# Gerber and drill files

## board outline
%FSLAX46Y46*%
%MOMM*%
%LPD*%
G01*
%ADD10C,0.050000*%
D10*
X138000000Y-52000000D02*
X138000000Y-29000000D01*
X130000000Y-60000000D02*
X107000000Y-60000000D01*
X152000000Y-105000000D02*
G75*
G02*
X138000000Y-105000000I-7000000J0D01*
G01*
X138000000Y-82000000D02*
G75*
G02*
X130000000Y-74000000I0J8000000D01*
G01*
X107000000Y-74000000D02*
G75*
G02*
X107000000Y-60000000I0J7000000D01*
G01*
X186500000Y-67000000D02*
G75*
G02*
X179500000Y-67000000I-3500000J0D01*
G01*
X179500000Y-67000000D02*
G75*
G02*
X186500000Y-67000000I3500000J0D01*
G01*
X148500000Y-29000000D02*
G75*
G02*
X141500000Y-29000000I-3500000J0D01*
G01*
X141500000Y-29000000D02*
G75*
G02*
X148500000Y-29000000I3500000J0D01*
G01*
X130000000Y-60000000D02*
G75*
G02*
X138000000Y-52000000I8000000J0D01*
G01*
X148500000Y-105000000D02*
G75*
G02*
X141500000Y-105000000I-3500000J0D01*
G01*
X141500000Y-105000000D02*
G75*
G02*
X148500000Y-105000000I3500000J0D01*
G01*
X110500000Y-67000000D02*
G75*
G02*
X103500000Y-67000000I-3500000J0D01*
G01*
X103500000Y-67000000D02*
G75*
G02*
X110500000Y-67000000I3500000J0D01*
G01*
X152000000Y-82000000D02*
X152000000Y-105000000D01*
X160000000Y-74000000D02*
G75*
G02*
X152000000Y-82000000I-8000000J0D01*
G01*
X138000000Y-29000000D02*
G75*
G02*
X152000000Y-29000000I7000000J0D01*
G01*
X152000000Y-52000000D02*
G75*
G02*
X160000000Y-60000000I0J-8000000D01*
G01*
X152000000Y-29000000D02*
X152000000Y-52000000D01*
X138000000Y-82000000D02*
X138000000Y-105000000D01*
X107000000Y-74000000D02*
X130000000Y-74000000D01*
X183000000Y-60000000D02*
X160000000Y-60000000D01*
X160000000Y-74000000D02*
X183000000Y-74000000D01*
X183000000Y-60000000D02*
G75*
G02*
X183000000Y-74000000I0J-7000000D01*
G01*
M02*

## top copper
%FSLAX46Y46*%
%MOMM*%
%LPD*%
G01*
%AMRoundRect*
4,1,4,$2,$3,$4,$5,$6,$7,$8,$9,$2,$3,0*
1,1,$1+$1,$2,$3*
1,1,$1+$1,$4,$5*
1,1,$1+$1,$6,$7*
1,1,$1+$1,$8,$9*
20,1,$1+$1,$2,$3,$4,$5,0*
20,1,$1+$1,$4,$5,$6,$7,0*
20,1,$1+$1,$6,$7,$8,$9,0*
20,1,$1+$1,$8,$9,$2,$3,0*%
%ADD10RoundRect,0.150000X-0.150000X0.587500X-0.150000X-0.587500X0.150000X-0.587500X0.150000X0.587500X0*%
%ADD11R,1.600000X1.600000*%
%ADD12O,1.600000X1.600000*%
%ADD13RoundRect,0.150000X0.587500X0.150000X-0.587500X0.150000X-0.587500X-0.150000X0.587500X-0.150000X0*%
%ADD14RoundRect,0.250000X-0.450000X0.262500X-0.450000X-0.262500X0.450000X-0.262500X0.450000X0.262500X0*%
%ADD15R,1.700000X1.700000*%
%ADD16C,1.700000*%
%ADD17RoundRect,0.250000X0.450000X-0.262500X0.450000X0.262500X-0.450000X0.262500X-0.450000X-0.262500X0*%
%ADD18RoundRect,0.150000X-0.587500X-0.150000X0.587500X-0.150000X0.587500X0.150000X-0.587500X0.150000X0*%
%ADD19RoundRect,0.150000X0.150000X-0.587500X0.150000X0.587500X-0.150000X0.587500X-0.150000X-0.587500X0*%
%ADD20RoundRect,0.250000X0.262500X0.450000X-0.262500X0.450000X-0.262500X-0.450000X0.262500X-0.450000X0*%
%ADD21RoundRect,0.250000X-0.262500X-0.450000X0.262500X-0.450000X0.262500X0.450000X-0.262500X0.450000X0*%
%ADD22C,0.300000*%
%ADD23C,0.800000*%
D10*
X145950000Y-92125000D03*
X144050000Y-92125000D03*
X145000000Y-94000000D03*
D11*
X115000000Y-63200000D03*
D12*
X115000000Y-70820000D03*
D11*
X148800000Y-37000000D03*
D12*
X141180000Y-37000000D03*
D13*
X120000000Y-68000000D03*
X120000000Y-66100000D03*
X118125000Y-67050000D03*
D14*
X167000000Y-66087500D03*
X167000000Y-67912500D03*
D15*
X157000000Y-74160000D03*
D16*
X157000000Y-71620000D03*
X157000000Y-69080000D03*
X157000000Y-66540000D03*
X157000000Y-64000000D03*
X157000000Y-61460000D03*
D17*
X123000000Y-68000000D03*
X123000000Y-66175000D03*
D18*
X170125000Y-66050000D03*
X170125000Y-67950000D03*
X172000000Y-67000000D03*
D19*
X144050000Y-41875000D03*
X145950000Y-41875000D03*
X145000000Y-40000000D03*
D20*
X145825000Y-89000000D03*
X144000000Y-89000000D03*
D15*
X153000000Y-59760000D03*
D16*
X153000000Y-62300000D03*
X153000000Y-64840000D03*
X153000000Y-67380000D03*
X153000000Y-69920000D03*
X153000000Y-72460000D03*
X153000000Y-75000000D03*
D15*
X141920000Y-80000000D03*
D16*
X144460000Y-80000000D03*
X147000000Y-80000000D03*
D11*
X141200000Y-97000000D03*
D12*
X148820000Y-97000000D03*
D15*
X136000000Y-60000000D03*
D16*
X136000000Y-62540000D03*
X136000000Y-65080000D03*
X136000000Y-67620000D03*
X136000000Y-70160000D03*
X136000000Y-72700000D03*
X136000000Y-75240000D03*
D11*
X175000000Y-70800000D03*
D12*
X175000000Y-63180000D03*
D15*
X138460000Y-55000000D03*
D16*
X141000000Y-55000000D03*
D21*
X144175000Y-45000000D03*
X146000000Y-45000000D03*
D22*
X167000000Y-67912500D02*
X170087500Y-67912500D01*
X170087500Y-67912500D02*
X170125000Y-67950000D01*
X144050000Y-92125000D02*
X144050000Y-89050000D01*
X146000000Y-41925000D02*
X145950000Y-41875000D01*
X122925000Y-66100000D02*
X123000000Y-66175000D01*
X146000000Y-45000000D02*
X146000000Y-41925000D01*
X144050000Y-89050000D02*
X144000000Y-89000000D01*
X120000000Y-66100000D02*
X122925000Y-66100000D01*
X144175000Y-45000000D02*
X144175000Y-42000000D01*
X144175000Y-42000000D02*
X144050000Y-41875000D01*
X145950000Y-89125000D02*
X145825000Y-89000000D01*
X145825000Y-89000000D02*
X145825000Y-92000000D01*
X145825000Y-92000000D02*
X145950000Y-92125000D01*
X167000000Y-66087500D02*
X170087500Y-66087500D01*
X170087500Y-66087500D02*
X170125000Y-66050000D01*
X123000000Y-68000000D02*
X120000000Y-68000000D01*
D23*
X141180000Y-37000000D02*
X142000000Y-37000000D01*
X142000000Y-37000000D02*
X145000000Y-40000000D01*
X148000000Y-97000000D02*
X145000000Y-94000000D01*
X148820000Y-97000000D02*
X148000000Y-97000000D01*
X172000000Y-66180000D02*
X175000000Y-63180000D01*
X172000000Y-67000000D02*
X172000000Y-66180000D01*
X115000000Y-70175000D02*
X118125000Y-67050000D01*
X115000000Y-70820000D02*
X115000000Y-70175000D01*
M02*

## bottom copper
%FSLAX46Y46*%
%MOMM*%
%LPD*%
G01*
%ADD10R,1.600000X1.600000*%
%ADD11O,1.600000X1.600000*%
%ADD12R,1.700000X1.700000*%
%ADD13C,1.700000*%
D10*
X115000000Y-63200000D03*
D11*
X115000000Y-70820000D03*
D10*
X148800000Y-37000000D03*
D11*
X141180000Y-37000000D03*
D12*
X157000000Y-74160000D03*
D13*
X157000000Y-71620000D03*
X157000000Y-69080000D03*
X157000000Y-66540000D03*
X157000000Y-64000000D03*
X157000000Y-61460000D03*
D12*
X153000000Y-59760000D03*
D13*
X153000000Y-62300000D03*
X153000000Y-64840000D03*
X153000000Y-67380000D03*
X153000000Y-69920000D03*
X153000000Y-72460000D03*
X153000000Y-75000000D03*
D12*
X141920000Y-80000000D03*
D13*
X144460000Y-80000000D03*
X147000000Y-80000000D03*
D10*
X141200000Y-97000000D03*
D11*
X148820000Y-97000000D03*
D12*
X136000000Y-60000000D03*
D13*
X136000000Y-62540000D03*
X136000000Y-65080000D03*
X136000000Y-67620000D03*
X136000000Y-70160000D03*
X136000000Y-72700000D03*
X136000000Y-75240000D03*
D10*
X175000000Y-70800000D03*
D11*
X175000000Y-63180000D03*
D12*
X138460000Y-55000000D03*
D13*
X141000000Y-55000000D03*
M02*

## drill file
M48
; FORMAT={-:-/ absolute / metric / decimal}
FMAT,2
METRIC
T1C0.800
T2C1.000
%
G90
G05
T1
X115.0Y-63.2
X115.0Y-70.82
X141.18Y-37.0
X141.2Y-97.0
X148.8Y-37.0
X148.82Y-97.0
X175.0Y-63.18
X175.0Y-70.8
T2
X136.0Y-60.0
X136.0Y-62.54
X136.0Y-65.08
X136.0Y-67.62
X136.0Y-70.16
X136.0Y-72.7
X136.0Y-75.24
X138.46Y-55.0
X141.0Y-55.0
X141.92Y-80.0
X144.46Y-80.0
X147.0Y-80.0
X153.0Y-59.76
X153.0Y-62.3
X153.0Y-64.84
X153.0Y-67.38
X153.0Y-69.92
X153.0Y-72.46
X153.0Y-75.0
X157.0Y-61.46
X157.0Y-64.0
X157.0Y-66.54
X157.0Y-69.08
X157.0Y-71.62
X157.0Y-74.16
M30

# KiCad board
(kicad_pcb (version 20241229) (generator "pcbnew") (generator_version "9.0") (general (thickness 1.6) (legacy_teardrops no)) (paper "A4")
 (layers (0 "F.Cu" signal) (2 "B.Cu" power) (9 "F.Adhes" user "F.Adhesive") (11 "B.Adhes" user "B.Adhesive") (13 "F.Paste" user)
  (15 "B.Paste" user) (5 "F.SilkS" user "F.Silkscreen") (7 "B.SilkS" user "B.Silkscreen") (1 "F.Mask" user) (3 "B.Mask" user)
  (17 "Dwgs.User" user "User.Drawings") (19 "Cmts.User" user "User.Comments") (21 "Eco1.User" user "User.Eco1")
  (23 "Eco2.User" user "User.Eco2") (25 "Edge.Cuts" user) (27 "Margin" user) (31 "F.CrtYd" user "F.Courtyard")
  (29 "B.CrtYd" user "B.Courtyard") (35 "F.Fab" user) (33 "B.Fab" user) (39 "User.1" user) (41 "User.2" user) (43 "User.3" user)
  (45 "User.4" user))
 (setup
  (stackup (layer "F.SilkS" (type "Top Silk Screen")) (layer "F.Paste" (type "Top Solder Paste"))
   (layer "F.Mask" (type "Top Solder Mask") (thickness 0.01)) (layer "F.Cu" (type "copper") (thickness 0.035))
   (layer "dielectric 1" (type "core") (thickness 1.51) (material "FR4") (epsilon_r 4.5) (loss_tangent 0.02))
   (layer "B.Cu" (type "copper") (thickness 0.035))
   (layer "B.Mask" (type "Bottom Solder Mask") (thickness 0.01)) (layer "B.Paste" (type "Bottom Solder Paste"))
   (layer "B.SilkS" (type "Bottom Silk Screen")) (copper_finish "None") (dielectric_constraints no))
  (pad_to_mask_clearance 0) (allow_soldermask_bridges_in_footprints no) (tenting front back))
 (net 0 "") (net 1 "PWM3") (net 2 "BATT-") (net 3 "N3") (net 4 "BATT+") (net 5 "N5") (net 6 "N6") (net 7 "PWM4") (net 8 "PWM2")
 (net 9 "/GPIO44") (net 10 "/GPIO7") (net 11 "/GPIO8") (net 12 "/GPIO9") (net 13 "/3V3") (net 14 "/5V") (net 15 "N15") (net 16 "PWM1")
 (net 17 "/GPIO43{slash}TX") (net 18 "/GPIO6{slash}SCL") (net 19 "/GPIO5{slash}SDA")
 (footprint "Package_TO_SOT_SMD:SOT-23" (layer "F.Cu") (at 145 93.0625 -90)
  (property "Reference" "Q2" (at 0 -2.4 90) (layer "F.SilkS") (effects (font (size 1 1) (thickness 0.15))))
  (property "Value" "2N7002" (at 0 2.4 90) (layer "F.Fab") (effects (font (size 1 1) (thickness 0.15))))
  (pad "1" smd roundrect (at -0.9375 -0.95 270) (size 1.475 0.6) (layers "F.Cu" "F.Mask" "F.Paste") (roundrect_rratio 0.25) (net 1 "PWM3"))
  (pad "2" smd roundrect (at -0.9375 0.95 270) (size 1.475 0.6) (layers "F.Cu" "F.Mask" "F.Paste") (roundrect_rratio 0.25) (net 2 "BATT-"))
  (pad "3" smd roundrect (at 0.9375 0 270) (size 1.475 0.6) (layers "F.Cu" "F.Mask" "F.Paste") (roundrect_rratio 0.25) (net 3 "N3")))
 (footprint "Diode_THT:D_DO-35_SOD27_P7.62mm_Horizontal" (layer "F.Cu") (at 115 63.2 -90)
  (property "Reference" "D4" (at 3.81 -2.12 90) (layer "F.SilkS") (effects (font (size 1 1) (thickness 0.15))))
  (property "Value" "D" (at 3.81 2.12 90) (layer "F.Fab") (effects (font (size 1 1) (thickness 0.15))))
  (pad "1" thru_hole rect (at 0 0 270) (size 1.6 1.6) (drill 0.8) (layers "*.Cu" "*.Mask") (remove_unused_layers no) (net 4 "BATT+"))
  (pad "2" thru_hole oval (at 7.62 0 270) (size 1.6 1.6) (drill 0.8) (layers "*.Cu" "*.Mask") (remove_unused_layers no) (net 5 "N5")))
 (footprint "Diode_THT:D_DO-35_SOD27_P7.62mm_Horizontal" (layer "F.Cu") (at 148.8 37 180)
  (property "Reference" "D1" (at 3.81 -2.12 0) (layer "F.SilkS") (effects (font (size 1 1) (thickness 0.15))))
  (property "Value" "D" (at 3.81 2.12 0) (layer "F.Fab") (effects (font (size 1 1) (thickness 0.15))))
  (pad "1" thru_hole rect (at 0 0 180) (size 1.6 1.6) (drill 0.8) (layers "*.Cu" "*.Mask") (remove_unused_layers no) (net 4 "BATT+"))
  (pad "2" thru_hole oval (at 7.62 0 180) (size 1.6 1.6) (drill 0.8) (layers "*.Cu" "*.Mask") (remove_unused_layers no) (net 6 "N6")))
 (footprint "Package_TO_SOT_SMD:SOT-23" (layer "F.Cu") (at 119.0625 67.05 180)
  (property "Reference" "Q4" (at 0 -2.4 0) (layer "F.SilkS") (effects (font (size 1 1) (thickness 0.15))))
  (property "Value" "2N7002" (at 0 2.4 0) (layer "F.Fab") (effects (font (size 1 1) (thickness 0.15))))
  (pad "1" smd roundrect (at -0.9375 -0.95 180) (size 1.475 0.6) (layers "F.Cu" "F.Mask" "F.Paste") (roundrect_rratio 0.25) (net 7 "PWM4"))
  (pad "2" smd roundrect (at -0.9375 0.95 180) (size 1.475 0.6) (layers "F.Cu" "F.Mask" "F.Paste") (roundrect_rratio 0.25) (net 2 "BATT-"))
  (pad "3" smd roundrect (at 0.9375 0 180) (size 1.475 0.6) (layers "F.Cu" "F.Mask" "F.Paste") (roundrect_rratio 0.25) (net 5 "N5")))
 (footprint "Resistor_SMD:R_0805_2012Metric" (layer "F.Cu") (at 167 67 -90)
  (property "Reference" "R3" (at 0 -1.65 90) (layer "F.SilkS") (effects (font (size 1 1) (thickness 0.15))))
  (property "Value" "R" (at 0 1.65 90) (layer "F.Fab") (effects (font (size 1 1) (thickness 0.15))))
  (pad "1" smd roundrect (at -0.9125 0 270) (size 1.025 1.4) (layers "F.Cu" "F.Mask" "F.Paste") (roundrect_rratio 0.243902) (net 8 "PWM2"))
  (pad "2" smd roundrect (at 0.9125 0 270) (size 1.025 1.4) (layers "F.Cu" "F.Mask" "F.Paste") (roundrect_rratio 0.243902) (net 2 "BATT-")))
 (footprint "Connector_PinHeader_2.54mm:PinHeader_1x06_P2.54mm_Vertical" (layer "F.Cu") (at 157 74.16 180)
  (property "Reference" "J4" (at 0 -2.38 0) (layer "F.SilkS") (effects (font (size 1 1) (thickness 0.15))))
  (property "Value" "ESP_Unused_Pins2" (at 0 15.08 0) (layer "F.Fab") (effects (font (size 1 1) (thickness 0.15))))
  (pad "1" thru_hole rect (at 0 0 180) (size 1.7 1.7) (drill 1) (layers "*.Cu" "*.Mask") (remove_unused_layers no) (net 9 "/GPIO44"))
  (pad "2" thru_hole circle (at 0 2.54 180) (size 1.7 1.7) (drill 1) (layers "*.Cu" "*.Mask") (remove_unused_layers no) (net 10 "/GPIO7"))
  (pad "3" thru_hole circle (at 0 5.08 180) (size 1.7 1.7) (drill 1) (layers "*.Cu" "*.Mask") (remove_unused_layers no) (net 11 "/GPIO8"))
  (pad "4" thru_hole circle (at 0 7.62 180) (size 1.7 1.7) (drill 1) (layers "*.Cu" "*.Mask") (remove_unused_layers no) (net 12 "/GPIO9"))
  (pad "5" thru_hole circle (at 0 10.16 180) (size 1.7 1.7) (drill 1) (layers "*.Cu" "*.Mask") (remove_unused_layers no) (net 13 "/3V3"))
  (pad "6" thru_hole circle (at 0 12.7 180) (size 1.7 1.7) (drill 1) (layers "*.Cu" "*.Mask") (remove_unused_layers no) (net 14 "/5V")))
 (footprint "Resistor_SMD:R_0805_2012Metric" (layer "F.Cu") (at 123 67.0875 90)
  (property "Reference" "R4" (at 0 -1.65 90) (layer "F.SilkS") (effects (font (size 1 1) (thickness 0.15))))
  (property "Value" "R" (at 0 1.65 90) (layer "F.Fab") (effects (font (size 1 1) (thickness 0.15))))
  (pad "1" smd roundrect (at -0.9125 0 90) (size 1.025 1.4) (layers "F.Cu" "F.Mask" "F.Paste") (roundrect_rratio 0.243902) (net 7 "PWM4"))
  (pad "2" smd roundrect (at 0.9125 0 90) (size 1.025 1.4) (layers "F.Cu" "F.Mask" "F.Paste") (roundrect_rratio 0.243902) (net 2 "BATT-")))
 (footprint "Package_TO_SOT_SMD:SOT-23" (layer "F.Cu") (at 171.0625 67)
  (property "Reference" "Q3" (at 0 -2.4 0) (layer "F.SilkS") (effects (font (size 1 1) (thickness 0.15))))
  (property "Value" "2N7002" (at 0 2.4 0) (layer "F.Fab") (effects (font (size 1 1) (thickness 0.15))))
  (pad "1" smd roundrect (at -0.9375 -0.95) (size 1.475 0.6) (layers "F.Cu" "F.Mask" "F.Paste") (roundrect_rratio 0.25) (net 8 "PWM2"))
  (pad "2" smd roundrect (at -0.9375 0.95) (size 1.475 0.6) (layers "F.Cu" "F.Mask" "F.Paste") (roundrect_rratio 0.25) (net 2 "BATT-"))
  (pad "3" smd roundrect (at 0.9375 0) (size 1.475 0.6) (layers "F.Cu" "F.Mask" "F.Paste") (roundrect_rratio 0.25) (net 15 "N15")))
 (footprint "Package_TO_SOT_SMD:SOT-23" (layer "F.Cu") (at 145 40.9375 90)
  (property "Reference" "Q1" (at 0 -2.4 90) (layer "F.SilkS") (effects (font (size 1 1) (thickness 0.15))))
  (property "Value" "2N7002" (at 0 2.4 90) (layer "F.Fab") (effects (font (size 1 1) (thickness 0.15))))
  (pad "1" smd roundrect (at -0.9375 -0.95 90) (size 1.475 0.6) (layers "F.Cu" "F.Mask" "F.Paste") (roundrect_rratio 0.25) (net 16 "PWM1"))
  (pad "2" smd roundrect (at -0.9375 0.95 90) (size 1.475 0.6) (layers "F.Cu" "F.Mask" "F.Paste") (roundrect_rratio 0.25) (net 2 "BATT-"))
  (pad "3" smd roundrect (at 0.9375 0 90) (size 1.475 0.6) (layers "F.Cu" "F.Mask" "F.Paste") (roundrect_rratio 0.25) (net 6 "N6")))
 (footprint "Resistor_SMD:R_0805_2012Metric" (layer "F.Cu") (at 144.9125 89 180)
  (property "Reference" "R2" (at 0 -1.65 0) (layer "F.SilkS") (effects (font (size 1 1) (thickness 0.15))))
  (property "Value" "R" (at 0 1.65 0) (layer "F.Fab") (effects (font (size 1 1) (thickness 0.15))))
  (pad "1" smd roundrect (at -0.9125 0 180) (size 1.025 1.4) (layers "F.Cu" "F.Mask" "F.Paste") (roundrect_rratio 0.243902) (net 1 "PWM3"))
  (pad "2" smd roundrect (at 0.9125 0 180) (size 1.025 1.4) (layers "F.Cu" "F.Mask" "F.Paste") (roundrect_rratio 0.243902) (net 2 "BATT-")))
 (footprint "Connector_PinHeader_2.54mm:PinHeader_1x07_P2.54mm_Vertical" (layer "F.Cu") (at 153 59.76)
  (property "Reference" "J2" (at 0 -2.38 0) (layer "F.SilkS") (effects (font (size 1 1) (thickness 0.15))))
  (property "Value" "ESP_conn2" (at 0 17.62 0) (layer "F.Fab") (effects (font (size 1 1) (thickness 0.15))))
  (pad "1" thru_hole rect (at 0 0) (size 1.7 1.7) (drill 1) (layers "*.Cu" "*.Mask") (remove_unused_layers no) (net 14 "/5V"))
  (pad "2" thru_hole circle (at 0 2.54) (size 1.7 1.7) (drill 1) (layers "*.Cu" "*.Mask") (remove_unused_layers no) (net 2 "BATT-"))
  (pad "3" thru_hole circle (at 0 5.08) (size 1.7 1.7) (drill 1) (layers "*.Cu" "*.Mask") (remove_unused_layers no) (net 13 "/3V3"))
  (pad "4" thru_hole circle (at 0 7.62) (size 1.7 1.7) (drill 1) (layers "*.Cu" "*.Mask") (remove_unused_layers no) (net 12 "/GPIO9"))
  (pad "5" thru_hole circle (at 0 10.16) (size 1.7 1.7) (drill 1) (layers "*.Cu" "*.Mask") (remove_unused_layers no) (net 11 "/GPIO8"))
  (pad "6" thru_hole circle (at 0 12.7) (size 1.7 1.7) (drill 1) (layers "*.Cu" "*.Mask") (remove_unused_layers no) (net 10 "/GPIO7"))
  (pad "7" thru_hole circle (at 0 15.24) (size 1.7 1.7) (drill 1) (layers "*.Cu" "*.Mask") (remove_unused_layers no) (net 9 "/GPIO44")))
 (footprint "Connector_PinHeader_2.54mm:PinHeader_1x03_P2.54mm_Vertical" (layer "F.Cu") (at 141.92 80 90)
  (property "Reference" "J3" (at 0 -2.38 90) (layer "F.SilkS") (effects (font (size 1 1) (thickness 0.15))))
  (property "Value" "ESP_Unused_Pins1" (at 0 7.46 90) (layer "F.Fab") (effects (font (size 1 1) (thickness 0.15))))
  (pad "1" thru_hole rect (at 0 0 90) (size 1.7 1.7) (drill 1) (layers "*.Cu" "*.Mask") (remove_unused_layers no)
   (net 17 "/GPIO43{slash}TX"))
  (pad "2" thru_hole circle (at 0 2.54 90) (size 1.7 1.7) (drill 1) (layers "*.Cu" "*.Mask") (remove_unused_layers no)
   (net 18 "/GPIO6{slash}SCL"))
  (pad "3" thru_hole circle (at 0 5.08 90) (size 1.7 1.7) (drill 1) (layers "*.Cu" "*.Mask") (remove_unused_layers no)
   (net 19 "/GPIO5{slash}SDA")))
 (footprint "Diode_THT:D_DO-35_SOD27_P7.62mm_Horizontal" (layer "F.Cu") (at 141.2 97)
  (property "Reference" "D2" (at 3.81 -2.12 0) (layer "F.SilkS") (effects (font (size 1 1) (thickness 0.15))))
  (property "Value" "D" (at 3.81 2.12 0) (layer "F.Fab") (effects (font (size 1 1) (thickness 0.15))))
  (pad "1" thru_hole rect (at 0 0) (size 1.6 1.6) (drill 0.8) (layers "*.Cu" "*.Mask") (remove_unused_layers no) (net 4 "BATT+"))
  (pad "2" thru_hole oval (at 7.62 0) (size 1.6 1.6) (drill 0.8) (layers "*.Cu" "*.Mask") (remove_unused_layers no) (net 3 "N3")))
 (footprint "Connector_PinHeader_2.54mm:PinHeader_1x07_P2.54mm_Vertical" (layer "F.Cu") (at 136 60)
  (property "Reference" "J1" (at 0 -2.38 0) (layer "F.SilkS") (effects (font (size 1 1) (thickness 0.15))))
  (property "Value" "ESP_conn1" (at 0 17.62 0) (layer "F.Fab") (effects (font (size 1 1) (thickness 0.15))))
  (pad "1" thru_hole rect (at 0 0) (size 1.7 1.7) (drill 1) (layers "*.Cu" "*.Mask") (remove_unused_layers no) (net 16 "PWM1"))
  (pad "2" thru_hole circle (at 0 2.54) (size 1.7 1.7) (drill 1) (layers "*.Cu" "*.Mask") (remove_unused_layers no) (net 8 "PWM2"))
  (pad "3" thru_hole circle (at 0 5.08) (size 1.7 1.7) (drill 1) (layers "*.Cu" "*.Mask") (remove_unused_layers no) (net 1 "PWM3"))
  (pad "4" thru_hole circle (at 0 7.62) (size 1.7 1.7) (drill 1) (layers "*.Cu" "*.Mask") (remove_unused_layers no) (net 7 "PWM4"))
  (pad "5" thru_hole circle (at 0 10.16) (size 1.7 1.7) (drill 1) (layers "*.Cu" "*.Mask") (remove_unused_layers no)
   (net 19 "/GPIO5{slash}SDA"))
  (pad "6" thru_hole circle (at 0 12.7) (size 1.7 1.7) (drill 1) (layers "*.Cu" "*.Mask") (remove_unused_layers no)
   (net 18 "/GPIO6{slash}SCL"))
  (pad "7" thru_hole circle (at 0 15.24) (size 1.7 1.7) (drill 1) (layers "*.Cu" "*.Mask") (remove_unused_layers no)
   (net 17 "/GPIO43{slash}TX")))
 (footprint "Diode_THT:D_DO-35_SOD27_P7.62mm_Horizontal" (layer "F.Cu") (at 175 70.8 90)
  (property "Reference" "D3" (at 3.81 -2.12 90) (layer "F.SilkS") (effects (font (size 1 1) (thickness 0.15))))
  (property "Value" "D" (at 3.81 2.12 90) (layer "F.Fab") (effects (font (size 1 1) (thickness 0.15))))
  (pad "1" thru_hole rect (at 0 0 90) (size 1.6 1.6) (drill 0.8) (layers "*.Cu" "*.Mask") (remove_unused_layers no) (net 4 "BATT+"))
  (pad "2" thru_hole oval (at 7.62 0 90) (size 1.6 1.6) (drill 0.8) (layers "*.Cu" "*.Mask") (remove_unused_layers no) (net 15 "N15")))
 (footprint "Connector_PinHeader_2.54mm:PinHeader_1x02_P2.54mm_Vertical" (layer "F.Cu") (at 138.46 55 90)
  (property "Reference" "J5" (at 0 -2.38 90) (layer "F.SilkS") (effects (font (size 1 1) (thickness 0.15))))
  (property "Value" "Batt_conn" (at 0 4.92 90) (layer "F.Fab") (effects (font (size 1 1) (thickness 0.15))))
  (pad "1" thru_hole rect (at 0 0 90) (size 1.7 1.7) (drill 1) (layers "*.Cu" "*.Mask") (remove_unused_layers no) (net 2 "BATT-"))
  (pad "2" thru_hole circle (at 0 2.54 90) (size 1.7 1.7) (drill 1) (layers "*.Cu" "*.Mask") (remove_unused_layers no) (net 4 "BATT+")))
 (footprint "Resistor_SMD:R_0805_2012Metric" (layer "F.Cu") (at 145.0875 45)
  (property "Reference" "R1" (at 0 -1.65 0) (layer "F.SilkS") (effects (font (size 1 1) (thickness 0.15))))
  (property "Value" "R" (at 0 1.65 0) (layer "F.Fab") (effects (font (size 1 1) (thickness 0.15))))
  (pad "1" smd roundrect (at -0.9125 0) (size 1.025 1.4) (layers "F.Cu" "F.Mask" "F.Paste") (roundrect_rratio 0.243902) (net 16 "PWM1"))
  (pad "2" smd roundrect (at 0.9125 0) (size 1.025 1.4) (layers "F.Cu" "F.Mask" "F.Paste") (roundrect_rratio 0.243902) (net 2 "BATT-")))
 (gr_line (start 138 52) (end 138 29) (stroke (width 0.05) (type default)) (layer "Edge.Cuts"))
 (gr_line (start 130 60) (end 107 60) (stroke (width 0.05) (type default)) (layer "Edge.Cuts"))
 (gr_arc (start 152 105) (mid 145 112) (end 138 105) (stroke (width 0.05) (type default)) (layer "Edge.Cuts"))
 (gr_arc (start 138 82) (mid 132.343146 79.656854) (end 130 74) (stroke (width 0.05) (type default)) (layer "Edge.Cuts"))
 (gr_arc (start 107 74) (mid 100 67) (end 107 60) (stroke (width 0.05) (type default)) (layer "Edge.Cuts"))
 (gr_circle (center 183 67) (end 186.5 67) (stroke (width 0.05) (type solid)) (fill no) (layer "Edge.Cuts"))
 (gr_circle (center 145 29) (end 148.5 29) (stroke (width 0.05) (type solid)) (fill no) (layer "Edge.Cuts"))
 (gr_arc (start 130 60) (mid 132.343146 54.343146) (end 138 52) (stroke (width 0.05) (type default)) (layer "Edge.Cuts"))
 (gr_circle (center 145 105) (end 148.5 105) (stroke (width 0.05) (type solid)) (fill no) (layer "Edge.Cuts"))
 (gr_circle (center 107 67) (end 110.5 67) (stroke (width 0.05) (type solid)) (fill no) (layer "Edge.Cuts"))
 (gr_line (start 152 82) (end 152 105) (stroke (width 0.05) (type default)) (layer "Edge.Cuts"))
 (gr_arc (start 160 74) (mid 157.656854 79.656854) (end 152 82) (stroke (width 0.05) (type default)) (layer "Edge.Cuts"))
 (gr_arc (start 138 29) (mid 145 22) (end 152 29) (stroke (width 0.05) (type default)) (layer "Edge.Cuts"))
 (gr_arc (start 152 52) (mid 157.656854 54.343146) (end 160 60) (stroke (width 0.05) (type default)) (layer "Edge.Cuts"))
 (gr_line (start 152 29) (end 152 52) (stroke (width 0.05) (type default)) (layer "Edge.Cuts"))
 (gr_line (start 138 82) (end 138 105) (stroke (width 0.05) (type default)) (layer "Edge.Cuts"))
 (gr_line (start 107 74) (end 130 74) (stroke (width 0.05) (type default)) (layer "Edge.Cuts"))
 (gr_line (start 183 60) (end 160 60) (stroke (width 0.05) (type default)) (layer "Edge.Cuts"))
 (gr_line (start 160 74) (end 183 74) (stroke (width 0.05) (type default)) (layer "Edge.Cuts"))
 (gr_arc (start 183 60) (mid 190 67) (end 183 74) (stroke (width 0.05) (type default)) (layer "Edge.Cuts"))
 (segment (start 167 67.9125) (end 170.0875 67.9125) (width 0.3) (layer "F.Cu") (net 2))
 (segment (start 170.0875 67.9125) (end 170.125 67.95) (width 0.3) (layer "F.Cu") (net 2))
 (segment (start 144.05 92.125) (end 144.05 89.05) (width 0.3) (layer "F.Cu") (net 2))
 (segment (start 146 41.925) (end 145.95 41.875) (width 0.3) (layer "F.Cu") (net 2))
 (segment (start 122.925 66.1) (end 123 66.175) (width 0.3) (layer "F.Cu") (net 2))
 (segment (start 146 45) (end 146 41.925) (width 0.3) (layer "F.Cu") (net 2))
 (segment (start 144.05 89.05) (end 144 89) (width 0.3) (layer "F.Cu") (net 2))
 (segment (start 120 66.1) (end 122.925 66.1) (width 0.3) (layer "F.Cu") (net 2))
 (segment (start 144.175 45) (end 144.175 42) (width 0.3) (layer "F.Cu") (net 16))
 (segment (start 144.175 42) (end 144.05 41.875) (width 0.3) (layer "F.Cu") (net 16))
 (segment (start 145.95 89.125) (end 145.825 89) (width 0.3) (layer "F.Cu") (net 1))
 (segment (start 145.825 89) (end 145.825 92) (width 0.3) (layer "F.Cu") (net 1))
 (segment (start 145.825 92) (end 145.95 92.125) (width 0.3) (layer "F.Cu") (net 1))
 (segment (start 167 66.0875) (end 170.0875 66.0875) (width 0.3) (layer "F.Cu") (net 8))
 (segment (start 170.0875 66.0875) (end 170.125 66.05) (width 0.3) (layer "F.Cu") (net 8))
 (segment (start 123 68) (end 120 68) (width 0.3) (layer "F.Cu") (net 7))
 (segment (start 141.18 37) (end 142 37) (width 0.8) (layer "F.Cu") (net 6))
 (segment (start 142 37) (end 145 40) (width 0.8) (layer "F.Cu") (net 6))
 (segment (start 148 97) (end 145 94) (width 0.8) (layer "F.Cu") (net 3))
 (segment (start 148.82 97) (end 148 97) (width 0.8) (layer "F.Cu") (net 3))
 (segment (start 172 66.18) (end 175 63.18) (width 0.8) (layer "F.Cu") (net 15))
 (segment (start 172 67) (end 172 66.18) (width 0.8) (layer "F.Cu") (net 15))
 (segment (start 115 70.175) (end 118.125 67.05) (width 0.8) (layer "F.Cu") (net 5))
 (segment (start 115 70.82) (end 115 70.175) (width 0.8) (layer "F.Cu") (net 5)))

